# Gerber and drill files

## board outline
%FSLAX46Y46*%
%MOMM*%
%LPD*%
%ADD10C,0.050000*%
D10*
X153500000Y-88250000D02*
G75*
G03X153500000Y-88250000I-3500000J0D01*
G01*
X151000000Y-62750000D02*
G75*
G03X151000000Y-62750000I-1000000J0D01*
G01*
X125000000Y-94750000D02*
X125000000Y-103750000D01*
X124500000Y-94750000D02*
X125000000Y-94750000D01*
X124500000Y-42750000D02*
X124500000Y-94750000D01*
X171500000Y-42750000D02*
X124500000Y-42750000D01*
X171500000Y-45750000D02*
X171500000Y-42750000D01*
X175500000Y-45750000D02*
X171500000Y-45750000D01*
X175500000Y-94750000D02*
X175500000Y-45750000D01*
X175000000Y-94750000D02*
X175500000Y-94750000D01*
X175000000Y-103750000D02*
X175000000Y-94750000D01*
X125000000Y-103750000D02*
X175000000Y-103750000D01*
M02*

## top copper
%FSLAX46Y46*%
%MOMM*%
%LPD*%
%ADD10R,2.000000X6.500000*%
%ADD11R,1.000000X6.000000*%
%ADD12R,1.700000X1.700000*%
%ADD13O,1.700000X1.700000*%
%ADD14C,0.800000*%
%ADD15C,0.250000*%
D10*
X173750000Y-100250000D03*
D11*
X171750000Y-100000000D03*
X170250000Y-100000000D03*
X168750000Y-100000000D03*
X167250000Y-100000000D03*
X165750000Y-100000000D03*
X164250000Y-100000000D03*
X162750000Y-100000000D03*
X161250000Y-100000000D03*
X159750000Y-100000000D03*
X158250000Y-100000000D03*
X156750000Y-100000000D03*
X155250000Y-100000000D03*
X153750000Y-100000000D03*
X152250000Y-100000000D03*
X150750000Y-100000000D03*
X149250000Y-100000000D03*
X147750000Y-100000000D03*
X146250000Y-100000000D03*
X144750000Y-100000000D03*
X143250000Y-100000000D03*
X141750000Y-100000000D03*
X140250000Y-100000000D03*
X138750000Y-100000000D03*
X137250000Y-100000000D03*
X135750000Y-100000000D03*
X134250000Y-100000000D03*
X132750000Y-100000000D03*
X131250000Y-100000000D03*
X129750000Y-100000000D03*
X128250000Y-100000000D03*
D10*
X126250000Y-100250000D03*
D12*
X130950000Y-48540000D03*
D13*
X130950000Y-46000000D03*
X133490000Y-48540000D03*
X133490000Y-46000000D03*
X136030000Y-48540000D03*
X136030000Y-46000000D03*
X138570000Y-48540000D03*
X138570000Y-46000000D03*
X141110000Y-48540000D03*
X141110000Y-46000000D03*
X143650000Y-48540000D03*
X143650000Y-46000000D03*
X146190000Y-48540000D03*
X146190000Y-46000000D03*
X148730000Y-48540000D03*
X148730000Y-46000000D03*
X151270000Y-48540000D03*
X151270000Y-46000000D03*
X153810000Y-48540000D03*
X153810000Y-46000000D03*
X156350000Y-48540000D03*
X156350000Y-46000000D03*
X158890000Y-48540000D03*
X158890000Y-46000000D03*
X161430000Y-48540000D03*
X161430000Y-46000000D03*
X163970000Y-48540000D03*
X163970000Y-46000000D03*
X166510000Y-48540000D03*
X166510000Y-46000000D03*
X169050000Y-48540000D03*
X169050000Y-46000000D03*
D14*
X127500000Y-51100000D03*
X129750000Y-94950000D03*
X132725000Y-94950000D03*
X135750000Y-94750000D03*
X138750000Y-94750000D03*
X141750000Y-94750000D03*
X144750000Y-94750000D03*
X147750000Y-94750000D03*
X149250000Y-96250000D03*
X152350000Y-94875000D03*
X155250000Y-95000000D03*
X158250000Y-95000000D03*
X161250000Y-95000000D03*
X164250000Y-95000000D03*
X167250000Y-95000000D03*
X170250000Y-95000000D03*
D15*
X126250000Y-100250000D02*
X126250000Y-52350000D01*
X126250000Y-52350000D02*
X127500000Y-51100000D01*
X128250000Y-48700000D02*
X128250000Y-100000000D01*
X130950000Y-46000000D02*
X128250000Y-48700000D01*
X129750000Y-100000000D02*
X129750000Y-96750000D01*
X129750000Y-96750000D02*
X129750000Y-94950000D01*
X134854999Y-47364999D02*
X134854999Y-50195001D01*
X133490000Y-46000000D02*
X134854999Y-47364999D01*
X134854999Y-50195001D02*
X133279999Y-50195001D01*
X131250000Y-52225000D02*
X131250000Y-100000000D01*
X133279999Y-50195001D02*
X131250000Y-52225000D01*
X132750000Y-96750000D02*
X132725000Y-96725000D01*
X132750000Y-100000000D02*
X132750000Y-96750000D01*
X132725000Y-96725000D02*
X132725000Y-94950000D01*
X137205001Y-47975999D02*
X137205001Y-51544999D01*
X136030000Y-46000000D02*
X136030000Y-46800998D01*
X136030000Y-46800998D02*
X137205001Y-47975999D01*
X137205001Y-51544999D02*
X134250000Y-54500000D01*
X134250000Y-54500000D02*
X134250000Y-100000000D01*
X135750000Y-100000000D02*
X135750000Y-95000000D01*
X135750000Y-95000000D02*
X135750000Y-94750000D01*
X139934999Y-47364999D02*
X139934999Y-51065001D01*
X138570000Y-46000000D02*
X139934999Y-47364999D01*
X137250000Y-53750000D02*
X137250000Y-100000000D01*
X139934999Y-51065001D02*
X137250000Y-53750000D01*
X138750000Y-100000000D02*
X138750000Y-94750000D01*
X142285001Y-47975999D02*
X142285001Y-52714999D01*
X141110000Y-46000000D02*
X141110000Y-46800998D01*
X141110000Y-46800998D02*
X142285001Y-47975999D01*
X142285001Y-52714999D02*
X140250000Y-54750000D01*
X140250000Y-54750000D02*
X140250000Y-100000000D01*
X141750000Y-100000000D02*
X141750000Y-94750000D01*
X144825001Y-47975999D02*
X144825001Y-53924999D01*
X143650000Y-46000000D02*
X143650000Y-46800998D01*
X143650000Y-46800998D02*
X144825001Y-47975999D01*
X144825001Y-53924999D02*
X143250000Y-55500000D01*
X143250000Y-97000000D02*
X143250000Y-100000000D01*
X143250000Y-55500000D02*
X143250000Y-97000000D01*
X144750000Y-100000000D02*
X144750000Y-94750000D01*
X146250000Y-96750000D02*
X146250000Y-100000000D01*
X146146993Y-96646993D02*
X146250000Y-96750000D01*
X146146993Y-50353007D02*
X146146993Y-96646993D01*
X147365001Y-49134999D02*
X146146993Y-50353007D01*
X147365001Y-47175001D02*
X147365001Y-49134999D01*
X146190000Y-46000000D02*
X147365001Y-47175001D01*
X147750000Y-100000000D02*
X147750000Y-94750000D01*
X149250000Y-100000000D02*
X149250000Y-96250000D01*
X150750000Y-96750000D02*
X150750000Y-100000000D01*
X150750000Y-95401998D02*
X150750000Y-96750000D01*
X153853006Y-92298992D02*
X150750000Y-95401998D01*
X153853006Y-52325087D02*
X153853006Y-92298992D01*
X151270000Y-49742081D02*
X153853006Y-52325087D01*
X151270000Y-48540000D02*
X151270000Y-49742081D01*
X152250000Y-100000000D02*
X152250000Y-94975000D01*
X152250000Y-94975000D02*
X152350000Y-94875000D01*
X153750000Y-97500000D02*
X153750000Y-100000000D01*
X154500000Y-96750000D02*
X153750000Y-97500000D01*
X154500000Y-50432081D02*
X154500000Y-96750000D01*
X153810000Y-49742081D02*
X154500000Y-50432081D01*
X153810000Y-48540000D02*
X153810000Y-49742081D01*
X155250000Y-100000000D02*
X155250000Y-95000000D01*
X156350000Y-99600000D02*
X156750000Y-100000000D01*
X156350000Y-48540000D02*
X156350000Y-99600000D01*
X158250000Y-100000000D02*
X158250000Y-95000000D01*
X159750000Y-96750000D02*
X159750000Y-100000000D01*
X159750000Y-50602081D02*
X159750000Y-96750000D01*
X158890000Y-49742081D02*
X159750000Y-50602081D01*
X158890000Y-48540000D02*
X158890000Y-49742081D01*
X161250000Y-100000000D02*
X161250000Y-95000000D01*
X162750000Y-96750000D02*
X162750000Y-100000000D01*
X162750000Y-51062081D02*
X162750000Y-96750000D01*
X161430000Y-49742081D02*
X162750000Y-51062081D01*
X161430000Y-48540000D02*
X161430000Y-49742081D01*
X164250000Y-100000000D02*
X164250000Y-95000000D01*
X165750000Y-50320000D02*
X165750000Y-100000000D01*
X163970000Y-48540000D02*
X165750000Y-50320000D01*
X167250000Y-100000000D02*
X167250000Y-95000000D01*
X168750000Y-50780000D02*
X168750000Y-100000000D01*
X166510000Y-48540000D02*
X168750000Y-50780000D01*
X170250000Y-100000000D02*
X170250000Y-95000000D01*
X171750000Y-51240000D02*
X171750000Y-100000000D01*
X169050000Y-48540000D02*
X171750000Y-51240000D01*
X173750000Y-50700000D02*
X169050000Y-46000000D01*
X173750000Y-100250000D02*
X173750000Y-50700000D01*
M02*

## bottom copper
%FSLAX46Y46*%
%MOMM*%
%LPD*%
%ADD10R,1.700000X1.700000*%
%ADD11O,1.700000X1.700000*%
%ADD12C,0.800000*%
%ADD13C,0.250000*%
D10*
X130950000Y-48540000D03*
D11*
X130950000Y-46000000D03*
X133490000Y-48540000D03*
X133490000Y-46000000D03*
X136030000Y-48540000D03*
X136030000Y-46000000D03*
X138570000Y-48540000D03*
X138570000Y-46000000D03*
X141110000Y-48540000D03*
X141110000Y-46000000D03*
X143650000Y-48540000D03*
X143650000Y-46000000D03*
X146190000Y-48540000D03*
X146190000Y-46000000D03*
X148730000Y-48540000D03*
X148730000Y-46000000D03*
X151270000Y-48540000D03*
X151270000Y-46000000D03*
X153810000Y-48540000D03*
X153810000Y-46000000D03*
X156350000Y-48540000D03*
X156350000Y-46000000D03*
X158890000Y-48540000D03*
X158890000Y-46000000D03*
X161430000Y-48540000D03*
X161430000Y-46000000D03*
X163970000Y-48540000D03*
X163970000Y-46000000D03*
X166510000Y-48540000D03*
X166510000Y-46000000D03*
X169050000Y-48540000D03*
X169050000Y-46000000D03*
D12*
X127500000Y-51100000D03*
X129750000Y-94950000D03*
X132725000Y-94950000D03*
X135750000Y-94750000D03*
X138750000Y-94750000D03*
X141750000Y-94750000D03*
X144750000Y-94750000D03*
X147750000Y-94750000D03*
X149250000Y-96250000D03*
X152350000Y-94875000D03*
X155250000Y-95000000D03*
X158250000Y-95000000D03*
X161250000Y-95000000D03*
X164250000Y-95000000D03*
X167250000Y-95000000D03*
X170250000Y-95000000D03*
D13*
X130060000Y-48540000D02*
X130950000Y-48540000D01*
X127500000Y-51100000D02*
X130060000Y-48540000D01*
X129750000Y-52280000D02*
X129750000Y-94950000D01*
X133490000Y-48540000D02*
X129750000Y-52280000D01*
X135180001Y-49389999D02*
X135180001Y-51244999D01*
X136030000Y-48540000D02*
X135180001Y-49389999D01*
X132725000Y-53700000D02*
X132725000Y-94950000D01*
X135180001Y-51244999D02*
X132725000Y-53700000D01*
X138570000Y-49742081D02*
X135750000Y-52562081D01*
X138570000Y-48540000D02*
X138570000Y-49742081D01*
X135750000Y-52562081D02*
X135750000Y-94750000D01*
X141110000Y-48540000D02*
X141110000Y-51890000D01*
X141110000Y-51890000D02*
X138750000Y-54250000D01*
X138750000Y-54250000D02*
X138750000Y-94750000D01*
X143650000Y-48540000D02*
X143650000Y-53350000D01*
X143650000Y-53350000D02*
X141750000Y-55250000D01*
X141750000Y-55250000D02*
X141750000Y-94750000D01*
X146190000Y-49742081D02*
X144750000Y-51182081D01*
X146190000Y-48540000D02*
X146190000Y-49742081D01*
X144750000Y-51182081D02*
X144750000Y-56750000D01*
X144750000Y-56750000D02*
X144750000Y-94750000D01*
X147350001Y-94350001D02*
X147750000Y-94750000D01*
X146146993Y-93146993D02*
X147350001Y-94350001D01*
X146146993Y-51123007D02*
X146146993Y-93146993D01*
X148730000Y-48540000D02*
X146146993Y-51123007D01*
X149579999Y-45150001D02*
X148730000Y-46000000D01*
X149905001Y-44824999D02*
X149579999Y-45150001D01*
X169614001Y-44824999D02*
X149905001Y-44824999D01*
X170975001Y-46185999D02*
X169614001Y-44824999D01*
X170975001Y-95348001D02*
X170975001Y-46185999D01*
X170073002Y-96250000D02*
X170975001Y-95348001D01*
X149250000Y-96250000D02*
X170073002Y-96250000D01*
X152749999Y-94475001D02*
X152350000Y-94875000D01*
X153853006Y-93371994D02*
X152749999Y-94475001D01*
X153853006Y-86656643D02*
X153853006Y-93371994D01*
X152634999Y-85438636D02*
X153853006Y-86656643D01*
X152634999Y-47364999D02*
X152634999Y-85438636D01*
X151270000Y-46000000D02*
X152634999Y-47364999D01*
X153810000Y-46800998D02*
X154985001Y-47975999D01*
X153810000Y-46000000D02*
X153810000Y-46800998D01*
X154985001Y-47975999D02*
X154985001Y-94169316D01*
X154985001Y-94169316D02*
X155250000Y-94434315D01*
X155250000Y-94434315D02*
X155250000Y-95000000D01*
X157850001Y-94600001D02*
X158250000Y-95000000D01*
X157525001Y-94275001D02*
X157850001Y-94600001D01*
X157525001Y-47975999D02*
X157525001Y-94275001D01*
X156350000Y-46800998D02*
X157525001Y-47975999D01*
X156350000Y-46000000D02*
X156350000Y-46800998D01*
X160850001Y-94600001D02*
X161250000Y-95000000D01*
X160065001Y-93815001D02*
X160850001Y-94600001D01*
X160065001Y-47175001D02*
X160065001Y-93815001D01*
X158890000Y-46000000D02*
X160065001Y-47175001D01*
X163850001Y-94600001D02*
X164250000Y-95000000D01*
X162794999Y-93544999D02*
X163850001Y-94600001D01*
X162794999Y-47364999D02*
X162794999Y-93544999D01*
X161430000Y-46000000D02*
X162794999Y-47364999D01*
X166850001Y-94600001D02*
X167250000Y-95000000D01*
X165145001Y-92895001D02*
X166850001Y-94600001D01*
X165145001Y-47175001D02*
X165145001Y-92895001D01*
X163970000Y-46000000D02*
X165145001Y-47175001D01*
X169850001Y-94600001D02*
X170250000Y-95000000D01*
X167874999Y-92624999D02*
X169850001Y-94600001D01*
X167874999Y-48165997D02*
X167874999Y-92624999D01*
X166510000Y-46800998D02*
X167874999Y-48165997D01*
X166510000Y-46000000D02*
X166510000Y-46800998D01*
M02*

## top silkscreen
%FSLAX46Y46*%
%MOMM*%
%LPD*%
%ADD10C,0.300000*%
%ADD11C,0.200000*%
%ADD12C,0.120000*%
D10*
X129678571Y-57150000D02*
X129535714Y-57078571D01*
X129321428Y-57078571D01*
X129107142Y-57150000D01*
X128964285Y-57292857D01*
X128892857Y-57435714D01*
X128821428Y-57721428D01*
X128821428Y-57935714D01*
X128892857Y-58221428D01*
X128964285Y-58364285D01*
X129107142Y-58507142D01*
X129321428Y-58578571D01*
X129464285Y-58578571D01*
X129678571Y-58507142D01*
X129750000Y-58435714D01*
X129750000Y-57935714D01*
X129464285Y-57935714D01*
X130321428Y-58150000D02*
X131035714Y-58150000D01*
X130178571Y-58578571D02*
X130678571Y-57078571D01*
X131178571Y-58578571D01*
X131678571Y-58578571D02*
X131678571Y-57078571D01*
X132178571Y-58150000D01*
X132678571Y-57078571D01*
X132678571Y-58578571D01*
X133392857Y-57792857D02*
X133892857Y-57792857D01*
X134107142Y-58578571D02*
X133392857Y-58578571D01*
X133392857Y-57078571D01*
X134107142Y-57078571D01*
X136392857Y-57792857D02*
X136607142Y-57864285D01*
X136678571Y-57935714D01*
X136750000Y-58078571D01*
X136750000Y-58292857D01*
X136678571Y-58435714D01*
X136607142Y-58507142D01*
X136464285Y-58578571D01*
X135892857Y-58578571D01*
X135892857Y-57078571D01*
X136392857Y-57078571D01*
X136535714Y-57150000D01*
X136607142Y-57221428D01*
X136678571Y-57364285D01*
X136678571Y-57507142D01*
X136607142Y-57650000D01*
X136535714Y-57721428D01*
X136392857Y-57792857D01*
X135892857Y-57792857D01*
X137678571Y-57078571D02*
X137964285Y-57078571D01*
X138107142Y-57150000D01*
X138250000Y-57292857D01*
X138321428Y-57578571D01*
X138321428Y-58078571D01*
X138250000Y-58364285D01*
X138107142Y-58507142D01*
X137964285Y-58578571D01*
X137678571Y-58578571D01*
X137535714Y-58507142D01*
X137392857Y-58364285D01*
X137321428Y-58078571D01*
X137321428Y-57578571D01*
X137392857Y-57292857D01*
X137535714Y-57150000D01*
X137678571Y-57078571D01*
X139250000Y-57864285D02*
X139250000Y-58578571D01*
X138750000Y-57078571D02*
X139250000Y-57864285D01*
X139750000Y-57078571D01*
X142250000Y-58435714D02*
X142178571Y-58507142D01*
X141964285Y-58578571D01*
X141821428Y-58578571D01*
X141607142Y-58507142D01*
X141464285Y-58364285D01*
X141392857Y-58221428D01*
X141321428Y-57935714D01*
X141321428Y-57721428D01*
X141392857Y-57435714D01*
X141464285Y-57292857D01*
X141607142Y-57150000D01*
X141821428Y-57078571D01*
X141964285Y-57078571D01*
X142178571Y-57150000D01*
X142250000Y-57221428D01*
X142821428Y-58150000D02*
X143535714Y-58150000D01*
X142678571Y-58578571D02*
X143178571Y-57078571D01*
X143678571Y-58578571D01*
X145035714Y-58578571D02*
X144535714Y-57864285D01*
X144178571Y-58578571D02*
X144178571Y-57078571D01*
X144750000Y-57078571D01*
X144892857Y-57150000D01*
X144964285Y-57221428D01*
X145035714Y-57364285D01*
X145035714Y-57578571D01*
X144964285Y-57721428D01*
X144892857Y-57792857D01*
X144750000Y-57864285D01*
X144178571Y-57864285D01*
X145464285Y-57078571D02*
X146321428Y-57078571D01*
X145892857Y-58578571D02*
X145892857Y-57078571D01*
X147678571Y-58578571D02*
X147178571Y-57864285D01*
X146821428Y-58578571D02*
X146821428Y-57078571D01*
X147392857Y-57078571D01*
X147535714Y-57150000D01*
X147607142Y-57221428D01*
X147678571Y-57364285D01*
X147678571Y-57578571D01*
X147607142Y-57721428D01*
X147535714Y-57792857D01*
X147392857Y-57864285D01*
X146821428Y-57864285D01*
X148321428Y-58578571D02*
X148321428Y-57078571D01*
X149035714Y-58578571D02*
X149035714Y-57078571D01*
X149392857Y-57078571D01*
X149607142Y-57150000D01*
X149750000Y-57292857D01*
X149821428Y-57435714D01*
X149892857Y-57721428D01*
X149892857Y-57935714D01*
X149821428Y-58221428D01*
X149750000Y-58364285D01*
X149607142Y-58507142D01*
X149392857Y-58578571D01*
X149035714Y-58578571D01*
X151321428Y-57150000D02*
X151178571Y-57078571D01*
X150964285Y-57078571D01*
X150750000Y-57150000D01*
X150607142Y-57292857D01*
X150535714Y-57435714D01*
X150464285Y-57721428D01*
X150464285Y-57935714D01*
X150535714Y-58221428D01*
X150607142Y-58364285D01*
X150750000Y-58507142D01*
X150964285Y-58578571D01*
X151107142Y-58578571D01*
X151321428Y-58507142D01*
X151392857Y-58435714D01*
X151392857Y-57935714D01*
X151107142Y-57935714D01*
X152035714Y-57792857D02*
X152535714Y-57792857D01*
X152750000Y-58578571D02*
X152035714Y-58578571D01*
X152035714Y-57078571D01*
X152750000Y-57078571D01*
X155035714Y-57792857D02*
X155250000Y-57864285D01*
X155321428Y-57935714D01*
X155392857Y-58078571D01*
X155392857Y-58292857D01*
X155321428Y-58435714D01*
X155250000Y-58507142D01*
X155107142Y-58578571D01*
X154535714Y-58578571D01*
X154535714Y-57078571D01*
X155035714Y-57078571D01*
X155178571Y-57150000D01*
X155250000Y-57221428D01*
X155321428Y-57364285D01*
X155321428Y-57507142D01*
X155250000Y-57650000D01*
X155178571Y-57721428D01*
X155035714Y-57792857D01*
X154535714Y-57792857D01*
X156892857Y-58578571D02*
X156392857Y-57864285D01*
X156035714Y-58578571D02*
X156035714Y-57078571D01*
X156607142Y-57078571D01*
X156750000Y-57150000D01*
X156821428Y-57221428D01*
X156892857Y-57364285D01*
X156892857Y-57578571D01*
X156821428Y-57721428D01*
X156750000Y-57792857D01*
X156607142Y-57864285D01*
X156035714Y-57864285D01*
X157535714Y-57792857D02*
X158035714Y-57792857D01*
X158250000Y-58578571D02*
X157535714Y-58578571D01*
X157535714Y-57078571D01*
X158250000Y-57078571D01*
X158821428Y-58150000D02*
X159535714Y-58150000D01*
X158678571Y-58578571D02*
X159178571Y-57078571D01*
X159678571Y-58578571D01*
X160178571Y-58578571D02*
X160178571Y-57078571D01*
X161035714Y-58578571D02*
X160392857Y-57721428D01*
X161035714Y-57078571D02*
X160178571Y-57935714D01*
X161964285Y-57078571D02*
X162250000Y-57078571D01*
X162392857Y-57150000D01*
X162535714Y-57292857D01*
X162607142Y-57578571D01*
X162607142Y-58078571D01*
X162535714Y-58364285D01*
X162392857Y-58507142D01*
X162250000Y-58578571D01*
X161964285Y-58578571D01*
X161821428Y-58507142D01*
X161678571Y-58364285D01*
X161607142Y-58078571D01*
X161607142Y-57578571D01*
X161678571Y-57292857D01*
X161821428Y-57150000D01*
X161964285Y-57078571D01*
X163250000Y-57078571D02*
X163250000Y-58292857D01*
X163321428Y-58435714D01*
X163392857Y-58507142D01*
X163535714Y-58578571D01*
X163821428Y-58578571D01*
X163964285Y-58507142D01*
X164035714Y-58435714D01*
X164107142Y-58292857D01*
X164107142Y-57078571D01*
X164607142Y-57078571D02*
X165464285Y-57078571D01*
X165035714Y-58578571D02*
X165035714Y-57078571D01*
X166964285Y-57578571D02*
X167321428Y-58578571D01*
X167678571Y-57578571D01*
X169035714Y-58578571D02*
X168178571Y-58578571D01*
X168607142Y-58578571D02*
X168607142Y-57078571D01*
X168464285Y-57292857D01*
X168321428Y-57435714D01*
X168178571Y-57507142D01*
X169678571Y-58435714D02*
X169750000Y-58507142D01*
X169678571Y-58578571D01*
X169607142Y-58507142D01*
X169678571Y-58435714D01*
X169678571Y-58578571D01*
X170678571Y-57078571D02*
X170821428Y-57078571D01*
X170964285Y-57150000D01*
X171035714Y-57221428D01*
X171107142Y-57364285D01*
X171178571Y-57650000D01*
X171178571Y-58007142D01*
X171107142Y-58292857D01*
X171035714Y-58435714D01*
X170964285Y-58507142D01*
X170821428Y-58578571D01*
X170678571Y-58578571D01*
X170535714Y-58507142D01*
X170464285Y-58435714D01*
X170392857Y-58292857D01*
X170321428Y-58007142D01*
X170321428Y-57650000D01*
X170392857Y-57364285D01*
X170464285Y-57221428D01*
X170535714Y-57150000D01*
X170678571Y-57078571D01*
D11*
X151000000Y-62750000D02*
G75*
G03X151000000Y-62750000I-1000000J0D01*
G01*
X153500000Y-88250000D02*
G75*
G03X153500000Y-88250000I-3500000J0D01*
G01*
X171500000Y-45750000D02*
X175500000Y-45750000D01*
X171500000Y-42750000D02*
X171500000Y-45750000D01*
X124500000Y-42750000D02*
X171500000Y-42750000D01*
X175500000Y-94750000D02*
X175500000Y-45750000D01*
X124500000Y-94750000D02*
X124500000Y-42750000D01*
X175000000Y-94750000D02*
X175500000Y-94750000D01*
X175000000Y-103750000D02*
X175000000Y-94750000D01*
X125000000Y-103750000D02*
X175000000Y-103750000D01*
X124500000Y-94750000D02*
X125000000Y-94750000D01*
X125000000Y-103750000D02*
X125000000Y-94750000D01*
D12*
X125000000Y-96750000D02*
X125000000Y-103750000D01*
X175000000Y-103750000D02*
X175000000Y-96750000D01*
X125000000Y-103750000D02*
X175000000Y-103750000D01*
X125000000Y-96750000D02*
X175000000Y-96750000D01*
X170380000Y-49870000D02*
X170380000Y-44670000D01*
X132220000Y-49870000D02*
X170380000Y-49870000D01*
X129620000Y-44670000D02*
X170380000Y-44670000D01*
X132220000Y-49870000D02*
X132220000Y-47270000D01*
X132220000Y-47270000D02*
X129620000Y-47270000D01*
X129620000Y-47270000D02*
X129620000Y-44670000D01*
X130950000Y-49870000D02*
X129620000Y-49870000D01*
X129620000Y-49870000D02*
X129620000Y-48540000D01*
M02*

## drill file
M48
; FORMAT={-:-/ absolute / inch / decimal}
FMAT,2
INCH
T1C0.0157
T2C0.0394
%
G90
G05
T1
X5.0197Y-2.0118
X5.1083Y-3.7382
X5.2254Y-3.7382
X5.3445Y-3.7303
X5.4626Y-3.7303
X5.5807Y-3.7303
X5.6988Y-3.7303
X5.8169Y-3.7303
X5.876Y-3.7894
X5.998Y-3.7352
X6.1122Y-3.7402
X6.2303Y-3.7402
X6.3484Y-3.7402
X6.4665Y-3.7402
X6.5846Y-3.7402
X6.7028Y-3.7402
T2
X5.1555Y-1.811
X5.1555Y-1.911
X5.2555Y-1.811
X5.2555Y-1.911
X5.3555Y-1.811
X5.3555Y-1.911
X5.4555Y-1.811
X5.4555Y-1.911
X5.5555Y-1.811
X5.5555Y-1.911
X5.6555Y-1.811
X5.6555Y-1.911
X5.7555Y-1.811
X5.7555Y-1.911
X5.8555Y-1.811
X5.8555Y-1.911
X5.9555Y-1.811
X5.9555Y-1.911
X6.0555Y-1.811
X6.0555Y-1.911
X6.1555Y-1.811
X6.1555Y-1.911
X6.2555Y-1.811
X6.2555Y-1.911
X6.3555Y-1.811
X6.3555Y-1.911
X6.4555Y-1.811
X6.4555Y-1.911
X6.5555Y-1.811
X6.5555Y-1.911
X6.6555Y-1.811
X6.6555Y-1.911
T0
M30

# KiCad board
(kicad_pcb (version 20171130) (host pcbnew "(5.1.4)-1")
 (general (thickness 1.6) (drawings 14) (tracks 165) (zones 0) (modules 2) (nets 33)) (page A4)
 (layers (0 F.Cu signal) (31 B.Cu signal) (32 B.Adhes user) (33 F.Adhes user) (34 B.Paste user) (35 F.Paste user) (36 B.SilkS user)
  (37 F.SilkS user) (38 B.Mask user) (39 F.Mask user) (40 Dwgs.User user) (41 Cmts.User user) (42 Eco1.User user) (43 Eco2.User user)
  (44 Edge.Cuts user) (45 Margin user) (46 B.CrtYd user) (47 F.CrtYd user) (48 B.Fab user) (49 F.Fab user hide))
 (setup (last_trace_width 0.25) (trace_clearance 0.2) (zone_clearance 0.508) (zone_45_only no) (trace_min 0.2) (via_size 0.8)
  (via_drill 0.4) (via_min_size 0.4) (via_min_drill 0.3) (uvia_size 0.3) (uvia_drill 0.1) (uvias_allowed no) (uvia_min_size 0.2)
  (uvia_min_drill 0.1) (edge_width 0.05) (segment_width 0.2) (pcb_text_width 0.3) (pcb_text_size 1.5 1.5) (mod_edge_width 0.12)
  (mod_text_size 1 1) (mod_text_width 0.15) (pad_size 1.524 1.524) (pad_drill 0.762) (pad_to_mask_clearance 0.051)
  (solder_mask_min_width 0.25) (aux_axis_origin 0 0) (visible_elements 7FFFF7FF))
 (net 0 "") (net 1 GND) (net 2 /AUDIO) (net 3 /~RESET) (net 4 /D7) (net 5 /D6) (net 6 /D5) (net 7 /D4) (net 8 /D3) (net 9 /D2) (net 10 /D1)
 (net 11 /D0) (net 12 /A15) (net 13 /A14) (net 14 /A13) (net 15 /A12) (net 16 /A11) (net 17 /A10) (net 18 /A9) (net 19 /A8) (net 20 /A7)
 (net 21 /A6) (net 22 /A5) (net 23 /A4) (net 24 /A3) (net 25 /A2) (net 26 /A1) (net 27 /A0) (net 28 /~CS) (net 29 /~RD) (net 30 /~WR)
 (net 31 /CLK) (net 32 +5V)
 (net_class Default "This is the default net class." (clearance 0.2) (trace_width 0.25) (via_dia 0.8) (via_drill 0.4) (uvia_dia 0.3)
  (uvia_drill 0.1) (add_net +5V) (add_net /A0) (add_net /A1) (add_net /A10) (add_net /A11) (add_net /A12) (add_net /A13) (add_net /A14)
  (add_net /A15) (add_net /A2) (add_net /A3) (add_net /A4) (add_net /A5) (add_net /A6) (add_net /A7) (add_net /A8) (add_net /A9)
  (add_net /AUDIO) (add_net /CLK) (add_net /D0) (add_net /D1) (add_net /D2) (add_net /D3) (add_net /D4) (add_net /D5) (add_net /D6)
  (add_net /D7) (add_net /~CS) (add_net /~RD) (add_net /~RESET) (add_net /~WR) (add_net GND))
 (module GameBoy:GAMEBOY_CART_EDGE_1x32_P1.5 (layer F.Cu) (at 150 100)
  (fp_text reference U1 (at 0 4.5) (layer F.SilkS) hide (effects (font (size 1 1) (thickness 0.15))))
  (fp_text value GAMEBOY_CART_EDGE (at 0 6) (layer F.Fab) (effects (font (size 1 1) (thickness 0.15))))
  (fp_circle (center 0 -37.25) (end 1 -37.25) (layer F.SilkS) (width 0.2))
  (fp_circle (center 0 -11.75) (end 3.5 -11.75) (layer F.SilkS) (width 0.2))
  (fp_line (start 21.5 -54.25) (end 25.5 -54.25) (layer F.SilkS) (width 0.2))
  (fp_line (start 21.5 -57.25) (end 21.5 -54.25) (layer F.SilkS) (width 0.2))
  (fp_line (start -25.5 -57.25) (end 21.5 -57.25) (layer F.SilkS) (width 0.2))
  (fp_line (start 25.5 -5.25) (end 25.5 -54.25) (layer F.SilkS) (width 0.2))
  (fp_line (start -25.5 -5.25) (end -25.5 -57.25) (layer F.SilkS) (width 0.2))
  (fp_line (start 25 -5.25) (end 25.5 -5.25) (layer F.SilkS) (width 0.2))
  (fp_line (start 25 3.75) (end 25 -5.25) (layer F.SilkS) (width 0.2))
  (fp_line (start -25 3.75) (end 25 3.75) (layer F.SilkS) (width 0.2))
  (fp_line (start -25.5 -5.25) (end -25 -5.25) (layer F.SilkS) (width 0.2))
  (fp_line (start -25 3.75) (end -25 -5.25) (layer F.SilkS) (width 0.2))
  (fp_line (start -25 -3.25) (end -25 3.75) (layer F.SilkS) (width 0.12))
  (fp_line (start 25 3.75) (end 25 -3.25) (layer F.SilkS) (width 0.12))
  (fp_line (start -25 3.75) (end 25 3.75) (layer F.SilkS) (width 0.12))
  (fp_line (start -25 -3.25) (end 25 -3.25) (layer F.SilkS) (width 0.12))
  (pad 32 smd rect (at 23.75 0.25) (size 2 6.5) (layers F.Cu F.Paste F.Mask) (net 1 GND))
  (pad 31 smd rect (at 21.75 0) (size 1 6) (layers F.Cu F.Paste F.Mask) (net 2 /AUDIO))
  (pad 30 smd rect (at 20.25 0) (size 1 6) (layers F.Cu F.Paste F.Mask) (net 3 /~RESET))
  (pad 29 smd rect (at 18.75 0) (size 1 6) (layers F.Cu F.Paste F.Mask) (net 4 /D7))
  (pad 28 smd rect (at 17.25 0) (size 1 6) (layers F.Cu F.Paste F.Mask) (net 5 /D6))
  (pad 27 smd rect (at 15.75 0) (size 1 6) (layers F.Cu F.Paste F.Mask) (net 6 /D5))
  (pad 26 smd rect (at 14.25 0) (size 1 6) (layers F.Cu F.Paste F.Mask) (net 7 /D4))
  (pad 25 smd rect (at 12.75 0) (size 1 6) (layers F.Cu F.Paste F.Mask) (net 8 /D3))
  (pad 24 smd rect (at 11.25 0) (size 1 6) (layers F.Cu F.Paste F.Mask) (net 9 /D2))
  (pad 23 smd rect (at 9.75 0) (size 1 6) (layers F.Cu F.Paste F.Mask) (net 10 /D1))
  (pad 22 smd rect (at 8.25 0) (size 1 6) (layers F.Cu F.Paste F.Mask) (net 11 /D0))
  (pad 21 smd rect (at 6.75 0) (size 1 6) (layers F.Cu F.Paste F.Mask) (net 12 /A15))
  (pad 20 smd rect (at 5.25 0) (size 1 6) (layers F.Cu F.Paste F.Mask) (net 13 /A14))
  (pad 19 smd rect (at 3.75 0) (size 1 6) (layers F.Cu F.Paste F.Mask) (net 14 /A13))
  (pad 18 smd rect (at 2.25 0) (size 1 6) (layers F.Cu F.Paste F.Mask) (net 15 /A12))
  (pad 17 smd rect (at 0.75 0) (size 1 6) (layers F.Cu F.Paste F.Mask) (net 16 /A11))
  (pad 16 smd rect (at -0.75 0) (size 1 6) (layers F.Cu F.Paste F.Mask) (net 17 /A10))
  (pad 15 smd rect (at -2.25 0) (size 1 6) (layers F.Cu F.Paste F.Mask) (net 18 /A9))
  (pad 14 smd rect (at -3.75 0) (size 1 6) (layers F.Cu F.Paste F.Mask) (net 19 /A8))
  (pad 13 smd rect (at -5.25 0) (size 1 6) (layers F.Cu F.Paste F.Mask) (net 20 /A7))
  (pad 12 smd rect (at -6.75 0) (size 1 6) (layers F.Cu F.Paste F.Mask) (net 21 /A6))
  (pad 11 smd rect (at -8.25 0) (size 1 6) (layers F.Cu F.Paste F.Mask) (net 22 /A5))
  (pad 10 smd rect (at -9.75 0) (size 1 6) (layers F.Cu F.Paste F.Mask) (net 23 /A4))
  (pad 9 smd rect (at -11.25 0) (size 1 6) (layers F.Cu F.Paste F.Mask) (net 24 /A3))
  (pad 8 smd rect (at -12.75 0) (size 1 6) (layers F.Cu F.Paste F.Mask) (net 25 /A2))
  (pad 7 smd rect (at -14.25 0) (size 1 6) (layers F.Cu F.Paste F.Mask) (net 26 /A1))
  (pad 6 smd rect (at -15.75 0) (size 1 6) (layers F.Cu F.Paste F.Mask) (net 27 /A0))
  (pad 5 smd rect (at -17.25 0) (size 1 6) (layers F.Cu F.Paste F.Mask) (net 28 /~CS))
  (pad 4 smd rect (at -18.75 0) (size 1 6) (layers F.Cu F.Paste F.Mask) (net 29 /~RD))
  (pad 3 smd rect (at -20.25 0) (size 1 6) (layers F.Cu F.Paste F.Mask) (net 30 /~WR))
  (pad 2 smd rect (at -21.75 0) (size 1 6) (layers F.Cu F.Paste F.Mask) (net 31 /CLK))
  (pad 1 smd rect (at -23.75 0.25) (size 2 6.5) (layers F.Cu F.Paste F.Mask) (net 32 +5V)))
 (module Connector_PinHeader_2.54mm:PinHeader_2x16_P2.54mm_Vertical (layer F.Cu) (at 130.95 48.54 90)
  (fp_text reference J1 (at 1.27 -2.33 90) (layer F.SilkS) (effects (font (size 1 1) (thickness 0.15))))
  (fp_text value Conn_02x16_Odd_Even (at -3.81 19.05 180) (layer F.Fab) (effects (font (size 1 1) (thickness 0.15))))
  (fp_line (start -1.33 39.43) (end 3.87 39.43) (layer F.SilkS) (width 0.12))
  (fp_line (start -1.33 1.27) (end -1.33 39.43) (layer F.SilkS) (width 0.12))
  (fp_line (start 3.87 -1.33) (end 3.87 39.43) (layer F.SilkS) (width 0.12))
  (fp_line (start -1.33 1.27) (end 1.27 1.27) (layer F.SilkS) (width 0.12))
  (fp_line (start 1.27 1.27) (end 1.27 -1.33) (layer F.SilkS) (width 0.12))
  (fp_line (start 1.27 -1.33) (end 3.87 -1.33) (layer F.SilkS) (width 0.12))
  (fp_line (start -1.33 0) (end -1.33 -1.33) (layer F.SilkS) (width 0.12))
  (fp_line (start -1.33 -1.33) (end 0 -1.33) (layer F.SilkS) (width 0.12))
  (pad 1 thru_hole rect (at 0 0 90) (size 1.7 1.7) (drill 1) (layers *.Cu *.Mask) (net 32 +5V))
  (pad 2 thru_hole oval (at 2.54 0 90) (size 1.7 1.7) (drill 1) (layers *.Cu *.Mask) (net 31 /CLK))
  (pad 3 thru_hole oval (at 0 2.54 90) (size 1.7 1.7) (drill 1) (layers *.Cu *.Mask) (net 30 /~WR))
  (pad 4 thru_hole oval (at 2.54 2.54 90) (size 1.7 1.7) (drill 1) (layers *.Cu *.Mask) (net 29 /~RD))
  (pad 5 thru_hole oval (at 0 5.08 90) (size 1.7 1.7) (drill 1) (layers *.Cu *.Mask) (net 28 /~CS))
  (pad 6 thru_hole oval (at 2.54 5.08 90) (size 1.7 1.7) (drill 1) (layers *.Cu *.Mask) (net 27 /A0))
  (pad 7 thru_hole oval (at 0 7.62 90) (size 1.7 1.7) (drill 1) (layers *.Cu *.Mask) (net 26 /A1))
  (pad 8 thru_hole oval (at 2.54 7.62 90) (size 1.7 1.7) (drill 1) (layers *.Cu *.Mask) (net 25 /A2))
  (pad 9 thru_hole oval (at 0 10.16 90) (size 1.7 1.7) (drill 1) (layers *.Cu *.Mask) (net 24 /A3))
  (pad 10 thru_hole oval (at 2.54 10.16 90) (size 1.7 1.7) (drill 1) (layers *.Cu *.Mask) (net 23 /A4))
  (pad 11 thru_hole oval (at 0 12.7 90) (size 1.7 1.7) (drill 1) (layers *.Cu *.Mask) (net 22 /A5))
  (pad 12 thru_hole oval (at 2.54 12.7 90) (size 1.7 1.7) (drill 1) (layers *.Cu *.Mask) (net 21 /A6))
  (pad 13 thru_hole oval (at 0 15.24 90) (size 1.7 1.7) (drill 1) (layers *.Cu *.Mask) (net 20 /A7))
  (pad 14 thru_hole oval (at 2.54 15.24 90) (size 1.7 1.7) (drill 1) (layers *.Cu *.Mask) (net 19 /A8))
  (pad 15 thru_hole oval (at 0 17.78 90) (size 1.7 1.7) (drill 1) (layers *.Cu *.Mask) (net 18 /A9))
  (pad 16 thru_hole oval (at 2.54 17.78 90) (size 1.7 1.7) (drill 1) (layers *.Cu *.Mask) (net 17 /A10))
  (pad 17 thru_hole oval (at 0 20.32 90) (size 1.7 1.7) (drill 1) (layers *.Cu *.Mask) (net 16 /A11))
  (pad 18 thru_hole oval (at 2.54 20.32 90) (size 1.7 1.7) (drill 1) (layers *.Cu *.Mask) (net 15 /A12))
  (pad 19 thru_hole oval (at 0 22.86 90) (size 1.7 1.7) (drill 1) (layers *.Cu *.Mask) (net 14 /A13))
  (pad 20 thru_hole oval (at 2.54 22.86 90) (size 1.7 1.7) (drill 1) (layers *.Cu *.Mask) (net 13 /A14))
  (pad 21 thru_hole oval (at 0 25.4 90) (size 1.7 1.7) (drill 1) (layers *.Cu *.Mask) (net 12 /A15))
  (pad 22 thru_hole oval (at 2.54 25.4 90) (size 1.7 1.7) (drill 1) (layers *.Cu *.Mask) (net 11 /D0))
  (pad 23 thru_hole oval (at 0 27.94 90) (size 1.7 1.7) (drill 1) (layers *.Cu *.Mask) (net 10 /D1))
  (pad 24 thru_hole oval (at 2.54 27.94 90) (size 1.7 1.7) (drill 1) (layers *.Cu *.Mask) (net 9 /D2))
  (pad 25 thru_hole oval (at 0 30.48 90) (size 1.7 1.7) (drill 1) (layers *.Cu *.Mask) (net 8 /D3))
  (pad 26 thru_hole oval (at 2.54 30.48 90) (size 1.7 1.7) (drill 1) (layers *.Cu *.Mask) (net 7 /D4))
  (pad 27 thru_hole oval (at 0 33.02 90) (size 1.7 1.7) (drill 1) (layers *.Cu *.Mask) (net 6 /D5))
  (pad 28 thru_hole oval (at 2.54 33.02 90) (size 1.7 1.7) (drill 1) (layers *.Cu *.Mask) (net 5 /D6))
  (pad 29 thru_hole oval (at 0 35.56 90) (size 1.7 1.7) (drill 1) (layers *.Cu *.Mask) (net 4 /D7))
  (pad 30 thru_hole oval (at 2.54 35.56 90) (size 1.7 1.7) (drill 1) (layers *.Cu *.Mask) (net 3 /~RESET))
  (pad 31 thru_hole oval (at 0 38.1 90) (size 1.7 1.7) (drill 1) (layers *.Cu *.Mask) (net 2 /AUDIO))
  (pad 32 thru_hole oval (at 2.54 38.1 90) (size 1.7 1.7) (drill 1) (layers *.Cu *.Mask) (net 1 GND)))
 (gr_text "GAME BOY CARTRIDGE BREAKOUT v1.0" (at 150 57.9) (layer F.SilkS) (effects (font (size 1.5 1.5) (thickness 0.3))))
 (gr_circle (center 150 88.25) (end 153.5 88.25) (layer Edge.Cuts) (width 0.05))
 (gr_circle (center 150 62.75) (end 151 62.75) (layer Edge.Cuts) (width 0.05))
 (gr_line (start 125 94.75) (end 125 103.75) (layer Edge.Cuts) (width 0.05))
 (gr_line (start 124.5 94.75) (end 125 94.75) (layer Edge.Cuts) (width 0.05))
 (gr_line (start 124.5 42.75) (end 124.5 94.75) (layer Edge.Cuts) (width 0.05))
 (gr_line (start 171.5 42.75) (end 124.5 42.75) (layer Edge.Cuts) (width 0.05))
 (gr_line (start 171.5 45.75) (end 171.5 42.75) (layer Edge.Cuts) (width 0.05))
 (gr_line (start 175.5 45.75) (end 171.5 45.75) (layer Edge.Cuts) (width 0.05))
 (gr_line (start 175.5 94.75) (end 175.5 45.75) (layer Edge.Cuts) (width 0.05))
 (gr_line (start 175 94.75) (end 175.5 94.75) (layer Edge.Cuts) (width 0.05))
 (gr_line (start 175 103.75) (end 175 94.75) (layer Edge.Cuts) (width 0.05))
 (gr_line (start 125 103.75) (end 175 103.75) (layer Edge.Cuts) (width 0.05))
 (via (at 127.5 51.1) (size 0.8) (drill 0.4) (layers F.Cu B.Cu) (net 32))
 (segment (start 126.25 100.25) (end 126.25 52.35) (width 0.25) (layer F.Cu) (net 32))
 (segment (start 126.25 52.35) (end 127.5 51.1) (width 0.25) (layer F.Cu) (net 32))
 (segment (start 130.06 48.54) (end 130.95 48.54) (width 0.25) (layer B.Cu) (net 32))
 (segment (start 127.5 51.1) (end 130.06 48.54) (width 0.25) (layer B.Cu) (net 32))
 (segment (start 128.25 48.7) (end 128.25 100) (width 0.25) (layer F.Cu) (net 31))
 (segment (start 130.95 46) (end 128.25 48.7) (width 0.25) (layer F.Cu) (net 31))
 (segment (start 129.75 100) (end 129.75 96.75) (width 0.25) (layer F.Cu) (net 30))
 (via (at 129.75 94.95) (size 0.8) (drill 0.4) (layers F.Cu B.Cu) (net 30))
 (segment (start 129.75 96.75) (end 129.75 94.95) (width 0.25) (layer F.Cu) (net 30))
 (segment (start 129.75 52.28) (end 129.75 94.95) (width 0.25) (layer B.Cu) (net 30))
 (segment (start 133.49 48.54) (end 129.75 52.28) (width 0.25) (layer B.Cu) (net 30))
 (segment (start 134.854999 47.364999) (end 134.854999 50.195001) (width 0.25) (layer F.Cu) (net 29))
 (segment (start 133.49 46) (end 134.854999 47.364999) (width 0.25) (layer F.Cu) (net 29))
 (segment (start 134.854999 50.195001) (end 133.279999 50.195001) (width 0.25) (layer F.Cu) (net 29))
 (segment (start 131.25 52.225) (end 131.25 100) (width 0.25) (layer F.Cu) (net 29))
 (segment (start 133.279999 50.195001) (end 131.25 52.225) (width 0.25) (layer F.Cu) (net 29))
 (segment (start 132.75 96.75) (end 132.725 96.725) (width 0.25) (layer F.Cu) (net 28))
 (segment (start 132.75 100) (end 132.75 96.75) (width 0.25) (layer F.Cu) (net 28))
 (via (at 132.725 94.95) (size 0.8) (drill 0.4) (layers F.Cu B.Cu) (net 28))
 (segment (start 132.725 96.725) (end 132.725 94.95) (width 0.25) (layer F.Cu) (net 28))
 (segment (start 135.180001 49.389999) (end 135.180001 51.244999) (width 0.25) (layer B.Cu) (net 28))
 (segment (start 136.03 48.54) (end 135.180001 49.389999) (width 0.25) (layer B.Cu) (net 28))
 (segment (start 132.725 53.7) (end 132.725 94.95) (width 0.25) (layer B.Cu) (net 28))
 (segment (start 135.180001 51.244999) (end 132.725 53.7) (width 0.25) (layer B.Cu) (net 28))
 (segment (start 137.205001 47.975999) (end 137.205001 51.544999) (width 0.25) (layer F.Cu) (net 27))
 (segment (start 136.03 46) (end 136.03 46.800998) (width 0.25) (layer F.Cu) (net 27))
 (segment (start 136.03 46.800998) (end 137.205001 47.975999) (width 0.25) (layer F.Cu) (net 27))
 (segment (start 137.205001 51.544999) (end 134.25 54.5) (width 0.25) (layer F.Cu) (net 27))
 (segment (start 134.25 54.5) (end 134.25 100) (width 0.25) (layer F.Cu) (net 27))
 (segment (start 135.75 100) (end 135.75 95) (width 0.25) (layer F.Cu) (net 26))
 (via (at 135.75 94.75) (size 0.8) (drill 0.4) (layers F.Cu B.Cu) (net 26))
 (segment (start 135.75 95) (end 135.75 94.75) (width 0.25) (layer F.Cu) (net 26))
 (segment (start 138.57 49.742081) (end 135.75 52.562081) (width 0.25) (layer B.Cu) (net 26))
 (segment (start 138.57 48.54) (end 138.57 49.742081) (width 0.25) (layer B.Cu) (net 26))
 (segment (start 135.75 52.562081) (end 135.75 94.75) (width 0.25) (layer B.Cu) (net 26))
 (segment (start 139.934999 47.364999) (end 139.934999 51.065001) (width 0.25) (layer F.Cu) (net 25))
 (segment (start 138.57 46) (end 139.934999 47.364999) (width 0.25) (layer F.Cu) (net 25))
 (segment (start 137.25 53.75) (end 137.25 100) (width 0.25) (layer F.Cu) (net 25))
 (segment (start 139.934999 51.065001) (end 137.25 53.75) (width 0.25) (layer F.Cu) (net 25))
 (segment (start 138.75 100) (end 138.75 94.75) (width 0.25) (layer F.Cu) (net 24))
 (via (at 138.75 94.75) (size 0.8) (drill 0.4) (layers F.Cu B.Cu) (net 24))
 (segment (start 141.11 48.54) (end 141.11 51.89) (width 0.25) (layer B.Cu) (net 24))
 (segment (start 141.11 51.89) (end 138.75 54.25) (width 0.25) (layer B.Cu) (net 24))
 (segment (start 138.75 54.25) (end 138.75 94.75) (width 0.25) (layer B.Cu) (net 24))
 (segment (start 142.285001 47.975999) (end 142.285001 52.714999) (width 0.25) (layer F.Cu) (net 23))
 (segment (start 141.11 46) (end 141.11 46.800998) (width 0.25) (layer F.Cu) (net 23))
 (segment (start 141.11 46.800998) (end 142.285001 47.975999) (width 0.25) (layer F.Cu) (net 23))
 (segment (start 142.285001 52.714999) (end 140.25 54.75) (width 0.25) (layer F.Cu) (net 23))
 (segment (start 140.25 54.75) (end 140.25 100) (width 0.25) (layer F.Cu) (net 23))
 (segment (start 141.75 100) (end 141.75 94.75) (width 0.25) (layer F.Cu) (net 22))
 (via (at 141.75 94.75) (size 0.8) (drill 0.4) (layers F.Cu B.Cu) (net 22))
 (segment (start 143.65 48.54) (end 143.65 53.35) (width 0.25) (layer B.Cu) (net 22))
 (segment (start 143.65 53.35) (end 141.75 55.25) (width 0.25) (layer B.Cu) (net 22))
 (segment (start 141.75 55.25) (end 141.75 94.75) (width 0.25) (layer B.Cu) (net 22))
 (segment (start 144.825001 47.975999) (end 144.825001 53.924999) (width 0.25) (layer F.Cu) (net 21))
 (segment (start 143.65 46) (end 143.65 46.800998) (width 0.25) (layer F.Cu) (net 21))
 (segment (start 143.65 46.800998) (end 144.825001 47.975999) (width 0.25) (layer F.Cu) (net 21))
 (segment (start 144.825001 53.924999) (end 143.25 55.5) (width 0.25) (layer F.Cu) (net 21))
 (segment (start 143.25 97) (end 143.25 100) (width 0.25) (layer F.Cu) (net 21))
 (segment (start 143.25 55.5) (end 143.25 97) (width 0.25) (layer F.Cu) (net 21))
 (segment (start 144.75 100) (end 144.75 94.75) (width 0.25) (layer F.Cu) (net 20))
 (via (at 144.75 94.75) (size 0.8) (drill 0.4) (layers F.Cu B.Cu) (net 20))
 (segment (start 146.19 49.742081) (end 144.75 51.182081) (width 0.25) (layer B.Cu) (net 20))
 (segment (start 146.19 48.54) (end 146.19 49.742081) (width 0.25) (layer B.Cu) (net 20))
 (segment (start 144.75 51.182081) (end 144.75 56.75) (width 0.25) (layer B.Cu) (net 20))
 (segment (start 144.75 56.75) (end 144.75 94.75) (width 0.25) (layer B.Cu) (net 20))
 (segment (start 146.25 96.75) (end 146.25 100) (width 0.25) (layer F.Cu) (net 19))
 (segment (start 146.146993 96.646993) (end 146.25 96.75) (width 0.25) (layer F.Cu) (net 19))
 (segment (start 146.146993 50.353007) (end 146.146993 96.646993) (width 0.25) (layer F.Cu) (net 19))
 (segment (start 147.365001 49.134999) (end 146.146993 50.353007) (width 0.25) (layer F.Cu) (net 19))
 (segment (start 147.365001 47.175001) (end 147.365001 49.134999) (width 0.25) (layer F.Cu) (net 19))
 (segment (start 146.19 46) (end 147.365001 47.175001) (width 0.25) (layer F.Cu) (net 19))
 (segment (start 147.75 100) (end 147.75 94.75) (width 0.25) (layer F.Cu) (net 18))
 (via (at 147.75 94.75) (size 0.8) (drill 0.4) (layers F.Cu B.Cu) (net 18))
 (segment (start 147.350001 94.350001) (end 147.75 94.75) (width 0.25) (layer B.Cu) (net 18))
 (segment (start 146.146993 93.146993) (end 147.350001 94.350001) (width 0.25) (layer B.Cu) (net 18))
 (segment (start 146.146993 51.123007) (end 146.146993 93.146993) (width 0.25) (layer B.Cu) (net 18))
 (segment (start 148.73 48.54) (end 146.146993 51.123007) (width 0.25) (layer B.Cu) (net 18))
 (segment (start 149.25 100) (end 149.25 96.25) (width 0.25) (layer F.Cu) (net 17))
 (via (at 149.25 96.25) (size 0.8) (drill 0.4) (layers F.Cu B.Cu) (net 17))
 (segment (start 149.579999 45.150001) (end 148.73 46) (width 0.25) (layer B.Cu) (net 17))
 (segment (start 149.905001 44.824999) (end 149.579999 45.150001) (width 0.25) (layer B.Cu) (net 17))
 (segment (start 169.614001 44.824999) (end 149.905001 44.824999) (width 0.25) (layer B.Cu) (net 17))
 (segment (start 170.975001 46.185999) (end 169.614001 44.824999) (width 0.25) (layer B.Cu) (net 17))
 (segment (start 170.975001 95.348001) (end 170.975001 46.185999) (width 0.25) (layer B.Cu) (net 17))
 (segment (start 170.073002 96.25) (end 170.975001 95.348001) (width 0.25) (layer B.Cu) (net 17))
 (segment (start 149.25 96.25) (end 170.073002 96.25) (width 0.25) (layer B.Cu) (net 17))
 (segment (start 150.75 96.75) (end 150.75 100) (width 0.25) (layer F.Cu) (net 16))
 (segment (start 150.75 95.401998) (end 150.75 96.75) (width 0.25) (layer F.Cu) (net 16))
 (segment (start 153.853006 92.298992) (end 150.75 95.401998) (width 0.25) (layer F.Cu) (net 16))
 (segment (start 153.853006 52.325087) (end 153.853006 92.298992) (width 0.25) (layer F.Cu) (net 16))
 (segment (start 151.27 49.742081) (end 153.853006 52.325087) (width 0.25) (layer F.Cu) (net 16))
 (segment (start 151.27 48.54) (end 151.27 49.742081) (width 0.25) (layer F.Cu) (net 16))
 (via (at 152.35 94.875) (size 0.8) (drill 0.4) (layers F.Cu B.Cu) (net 15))
 (segment (start 152.25 100) (end 152.25 94.975) (width 0.25) (layer F.Cu) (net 15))
 (segment (start 152.25 94.975) (end 152.35 94.875) (width 0.25) (layer F.Cu) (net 15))
 (segment (start 152.749999 94.475001) (end 152.35 94.875) (width 0.25) (layer B.Cu) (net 15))
 (segment (start 153.853006 93.371994) (end 152.749999 94.475001) (width 0.25) (layer B.Cu) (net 15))
 (segment (start 153.853006 86.656643) (end 153.853006 93.371994) (width 0.25) (layer B.Cu) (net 15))
 (segment (start 152.634999 85.438636) (end 153.853006 86.656643) (width 0.25) (layer B.Cu) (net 15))
 (segment (start 152.634999 47.364999) (end 152.634999 85.438636) (width 0.25) (layer B.Cu) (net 15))
 (segment (start 151.27 46) (end 152.634999 47.364999) (width 0.25) (layer B.Cu) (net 15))
 (segment (start 153.75 97.5) (end 153.75 100) (width 0.25) (layer F.Cu) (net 14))
 (segment (start 154.5 96.75) (end 153.75 97.5) (width 0.25) (layer F.Cu) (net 14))
 (segment (start 154.5 50.432081) (end 154.5 96.75) (width 0.25) (layer F.Cu) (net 14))
 (segment (start 153.81 49.742081) (end 154.5 50.432081) (width 0.25) (layer F.Cu) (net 14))
 (segment (start 153.81 48.54) (end 153.81 49.742081) (width 0.25) (layer F.Cu) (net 14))
 (segment (start 155.25 100) (end 155.25 95) (width 0.25) (layer F.Cu) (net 13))
 (via (at 155.25 95) (size 0.8) (drill 0.4) (layers F.Cu B.Cu) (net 13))
 (segment (start 153.81 46.800998) (end 154.985001 47.975999) (width 0.25) (layer B.Cu) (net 13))
 (segment (start 153.81 46) (end 153.81 46.800998) (width 0.25) (layer B.Cu) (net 13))
 (segment (start 154.985001 47.975999) (end 154.985001 94.169316) (width 0.25) (layer B.Cu) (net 13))
 (segment (start 154.985001 94.169316) (end 155.25 94.434315) (width 0.25) (layer B.Cu) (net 13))
 (segment (start 155.25 94.434315) (end 155.25 95) (width 0.25) (layer B.Cu) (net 13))
 (segment (start 156.35 99.6) (end 156.75 100) (width 0.25) (layer F.Cu) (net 12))
 (segment (start 156.35 48.54) (end 156.35 99.6) (width 0.25) (layer F.Cu) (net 12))
 (via (at 158.25 95) (size 0.8) (drill 0.4) (layers F.Cu B.Cu) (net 11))
 (segment (start 158.25 100) (end 158.25 95) (width 0.25) (layer F.Cu) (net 11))
 (segment (start 157.850001 94.600001) (end 158.25 95) (width 0.25) (layer B.Cu) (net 11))
 (segment (start 157.525001 94.275001) (end 157.850001 94.600001) (width 0.25) (layer B.Cu) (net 11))
 (segment (start 157.525001 47.975999) (end 157.525001 94.275001) (width 0.25) (layer B.Cu) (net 11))
 (segment (start 156.35 46.800998) (end 157.525001 47.975999) (width 0.25) (layer B.Cu) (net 11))
 (segment (start 156.35 46) (end 156.35 46.800998) (width 0.25) (layer B.Cu) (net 11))
 (segment (start 159.75 96.75) (end 159.75 100) (width 0.25) (layer F.Cu) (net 10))
 (segment (start 159.75 50.602081) (end 159.75 96.75) (width 0.25) (layer F.Cu) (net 10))
 (segment (start 158.89 49.742081) (end 159.75 50.602081) (width 0.25) (layer F.Cu) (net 10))
 (segment (start 158.89 48.54) (end 158.89 49.742081) (width 0.25) (layer F.Cu) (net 10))
 (segment (start 161.25 100) (end 161.25 95) (width 0.25) (layer F.Cu) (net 9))
 (via (at 161.25 95) (size 0.8) (drill 0.4) (layers F.Cu B.Cu) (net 9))
 (segment (start 160.850001 94.600001) (end 161.25 95) (width 0.25) (layer B.Cu) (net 9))
 (segment (start 160.065001 93.815001) (end 160.850001 94.600001) (width 0.25) (layer B.Cu) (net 9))
 (segment (start 160.065001 47.175001) (end 160.065001 93.815001) (width 0.25) (layer B.Cu) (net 9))
 (segment (start 158.89 46) (end 160.065001 47.175001) (width 0.25) (layer B.Cu) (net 9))
 (segment (start 162.75 96.75) (end 162.75 100) (width 0.25) (layer F.Cu) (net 8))
 (segment (start 162.75 51.062081) (end 162.75 96.75) (width 0.25) (layer F.Cu) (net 8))
 (segment (start 161.43 49.742081) (end 162.75 51.062081) (width 0.25) (layer F.Cu) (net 8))
 (segment (start 161.43 48.54) (end 161.43 49.742081) (width 0.25) (layer F.Cu) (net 8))
 (via (at 164.25 95) (size 0.8) (drill 0.4) (layers F.Cu B.Cu) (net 7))
 (segment (start 164.25 100) (end 164.25 95) (width 0.25) (layer F.Cu) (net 7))
 (segment (start 163.850001 94.600001) (end 164.25 95) (width 0.25) (layer B.Cu) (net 7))
 (segment (start 162.794999 93.544999) (end 163.850001 94.600001) (width 0.25) (layer B.Cu) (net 7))
 (segment (start 162.794999 47.364999) (end 162.794999 93.544999) (width 0.25) (layer B.Cu) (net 7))
 (segment (start 161.43 46) (end 162.794999 47.364999) (width 0.25) (layer B.Cu) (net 7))
 (segment (start 165.75 50.32) (end 165.75 100) (width 0.25) (layer F.Cu) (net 6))
 (segment (start 163.97 48.54) (end 165.75 50.32) (width 0.25) (layer F.Cu) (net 6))
 (segment (start 167.25 100) (end 167.25 95) (width 0.25) (layer F.Cu) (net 5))
 (via (at 167.25 95) (size 0.8) (drill 0.4) (layers F.Cu B.Cu) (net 5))
 (segment (start 166.850001 94.600001) (end 167.25 95) (width 0.25) (layer B.Cu) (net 5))
 (segment (start 165.145001 92.895001) (end 166.850001 94.600001) (width 0.25) (layer B.Cu) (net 5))
 (segment (start 165.145001 47.175001) (end 165.145001 92.895001) (width 0.25) (layer B.Cu) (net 5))
 (segment (start 163.97 46) (end 165.145001 47.175001) (width 0.25) (layer B.Cu) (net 5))
 (segment (start 168.75 50.78) (end 168.75 100) (width 0.25) (layer F.Cu) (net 4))
 (segment (start 166.51 48.54) (end 168.75 50.78) (width 0.25) (layer F.Cu) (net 4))
 (via (at 170.25 95) (size 0.8) (drill 0.4) (layers F.Cu B.Cu) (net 3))
 (segment (start 170.25 100) (end 170.25 95) (width 0.25) (layer F.Cu) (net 3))
 (segment (start 169.850001 94.600001) (end 170.25 95) (width 0.25) (layer B.Cu) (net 3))
 (segment (start 167.874999 92.624999) (end 169.850001 94.600001) (width 0.25) (layer B.Cu) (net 3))
 (segment (start 167.874999 48.165997) (end 167.874999 92.624999) (width 0.25) (layer B.Cu) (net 3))
 (segment (start 166.51 46.800998) (end 167.874999 48.165997) (width 0.25) (layer B.Cu) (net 3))
 (segment (start 166.51 46) (end 166.51 46.800998) (width 0.25) (layer B.Cu) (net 3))
 (segment (start 171.75 51.24) (end 171.75 100) (width 0.25) (layer F.Cu) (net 2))
 (segment (start 169.05 48.54) (end 171.75 51.24) (width 0.25) (layer F.Cu) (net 2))
 (segment (start 173.75 50.7) (end 169.05 46) (width 0.25) (layer F.Cu) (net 1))
 (segment (start 173.75 100.25) (end 173.75 50.7) (width 0.25) (layer F.Cu) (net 1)))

